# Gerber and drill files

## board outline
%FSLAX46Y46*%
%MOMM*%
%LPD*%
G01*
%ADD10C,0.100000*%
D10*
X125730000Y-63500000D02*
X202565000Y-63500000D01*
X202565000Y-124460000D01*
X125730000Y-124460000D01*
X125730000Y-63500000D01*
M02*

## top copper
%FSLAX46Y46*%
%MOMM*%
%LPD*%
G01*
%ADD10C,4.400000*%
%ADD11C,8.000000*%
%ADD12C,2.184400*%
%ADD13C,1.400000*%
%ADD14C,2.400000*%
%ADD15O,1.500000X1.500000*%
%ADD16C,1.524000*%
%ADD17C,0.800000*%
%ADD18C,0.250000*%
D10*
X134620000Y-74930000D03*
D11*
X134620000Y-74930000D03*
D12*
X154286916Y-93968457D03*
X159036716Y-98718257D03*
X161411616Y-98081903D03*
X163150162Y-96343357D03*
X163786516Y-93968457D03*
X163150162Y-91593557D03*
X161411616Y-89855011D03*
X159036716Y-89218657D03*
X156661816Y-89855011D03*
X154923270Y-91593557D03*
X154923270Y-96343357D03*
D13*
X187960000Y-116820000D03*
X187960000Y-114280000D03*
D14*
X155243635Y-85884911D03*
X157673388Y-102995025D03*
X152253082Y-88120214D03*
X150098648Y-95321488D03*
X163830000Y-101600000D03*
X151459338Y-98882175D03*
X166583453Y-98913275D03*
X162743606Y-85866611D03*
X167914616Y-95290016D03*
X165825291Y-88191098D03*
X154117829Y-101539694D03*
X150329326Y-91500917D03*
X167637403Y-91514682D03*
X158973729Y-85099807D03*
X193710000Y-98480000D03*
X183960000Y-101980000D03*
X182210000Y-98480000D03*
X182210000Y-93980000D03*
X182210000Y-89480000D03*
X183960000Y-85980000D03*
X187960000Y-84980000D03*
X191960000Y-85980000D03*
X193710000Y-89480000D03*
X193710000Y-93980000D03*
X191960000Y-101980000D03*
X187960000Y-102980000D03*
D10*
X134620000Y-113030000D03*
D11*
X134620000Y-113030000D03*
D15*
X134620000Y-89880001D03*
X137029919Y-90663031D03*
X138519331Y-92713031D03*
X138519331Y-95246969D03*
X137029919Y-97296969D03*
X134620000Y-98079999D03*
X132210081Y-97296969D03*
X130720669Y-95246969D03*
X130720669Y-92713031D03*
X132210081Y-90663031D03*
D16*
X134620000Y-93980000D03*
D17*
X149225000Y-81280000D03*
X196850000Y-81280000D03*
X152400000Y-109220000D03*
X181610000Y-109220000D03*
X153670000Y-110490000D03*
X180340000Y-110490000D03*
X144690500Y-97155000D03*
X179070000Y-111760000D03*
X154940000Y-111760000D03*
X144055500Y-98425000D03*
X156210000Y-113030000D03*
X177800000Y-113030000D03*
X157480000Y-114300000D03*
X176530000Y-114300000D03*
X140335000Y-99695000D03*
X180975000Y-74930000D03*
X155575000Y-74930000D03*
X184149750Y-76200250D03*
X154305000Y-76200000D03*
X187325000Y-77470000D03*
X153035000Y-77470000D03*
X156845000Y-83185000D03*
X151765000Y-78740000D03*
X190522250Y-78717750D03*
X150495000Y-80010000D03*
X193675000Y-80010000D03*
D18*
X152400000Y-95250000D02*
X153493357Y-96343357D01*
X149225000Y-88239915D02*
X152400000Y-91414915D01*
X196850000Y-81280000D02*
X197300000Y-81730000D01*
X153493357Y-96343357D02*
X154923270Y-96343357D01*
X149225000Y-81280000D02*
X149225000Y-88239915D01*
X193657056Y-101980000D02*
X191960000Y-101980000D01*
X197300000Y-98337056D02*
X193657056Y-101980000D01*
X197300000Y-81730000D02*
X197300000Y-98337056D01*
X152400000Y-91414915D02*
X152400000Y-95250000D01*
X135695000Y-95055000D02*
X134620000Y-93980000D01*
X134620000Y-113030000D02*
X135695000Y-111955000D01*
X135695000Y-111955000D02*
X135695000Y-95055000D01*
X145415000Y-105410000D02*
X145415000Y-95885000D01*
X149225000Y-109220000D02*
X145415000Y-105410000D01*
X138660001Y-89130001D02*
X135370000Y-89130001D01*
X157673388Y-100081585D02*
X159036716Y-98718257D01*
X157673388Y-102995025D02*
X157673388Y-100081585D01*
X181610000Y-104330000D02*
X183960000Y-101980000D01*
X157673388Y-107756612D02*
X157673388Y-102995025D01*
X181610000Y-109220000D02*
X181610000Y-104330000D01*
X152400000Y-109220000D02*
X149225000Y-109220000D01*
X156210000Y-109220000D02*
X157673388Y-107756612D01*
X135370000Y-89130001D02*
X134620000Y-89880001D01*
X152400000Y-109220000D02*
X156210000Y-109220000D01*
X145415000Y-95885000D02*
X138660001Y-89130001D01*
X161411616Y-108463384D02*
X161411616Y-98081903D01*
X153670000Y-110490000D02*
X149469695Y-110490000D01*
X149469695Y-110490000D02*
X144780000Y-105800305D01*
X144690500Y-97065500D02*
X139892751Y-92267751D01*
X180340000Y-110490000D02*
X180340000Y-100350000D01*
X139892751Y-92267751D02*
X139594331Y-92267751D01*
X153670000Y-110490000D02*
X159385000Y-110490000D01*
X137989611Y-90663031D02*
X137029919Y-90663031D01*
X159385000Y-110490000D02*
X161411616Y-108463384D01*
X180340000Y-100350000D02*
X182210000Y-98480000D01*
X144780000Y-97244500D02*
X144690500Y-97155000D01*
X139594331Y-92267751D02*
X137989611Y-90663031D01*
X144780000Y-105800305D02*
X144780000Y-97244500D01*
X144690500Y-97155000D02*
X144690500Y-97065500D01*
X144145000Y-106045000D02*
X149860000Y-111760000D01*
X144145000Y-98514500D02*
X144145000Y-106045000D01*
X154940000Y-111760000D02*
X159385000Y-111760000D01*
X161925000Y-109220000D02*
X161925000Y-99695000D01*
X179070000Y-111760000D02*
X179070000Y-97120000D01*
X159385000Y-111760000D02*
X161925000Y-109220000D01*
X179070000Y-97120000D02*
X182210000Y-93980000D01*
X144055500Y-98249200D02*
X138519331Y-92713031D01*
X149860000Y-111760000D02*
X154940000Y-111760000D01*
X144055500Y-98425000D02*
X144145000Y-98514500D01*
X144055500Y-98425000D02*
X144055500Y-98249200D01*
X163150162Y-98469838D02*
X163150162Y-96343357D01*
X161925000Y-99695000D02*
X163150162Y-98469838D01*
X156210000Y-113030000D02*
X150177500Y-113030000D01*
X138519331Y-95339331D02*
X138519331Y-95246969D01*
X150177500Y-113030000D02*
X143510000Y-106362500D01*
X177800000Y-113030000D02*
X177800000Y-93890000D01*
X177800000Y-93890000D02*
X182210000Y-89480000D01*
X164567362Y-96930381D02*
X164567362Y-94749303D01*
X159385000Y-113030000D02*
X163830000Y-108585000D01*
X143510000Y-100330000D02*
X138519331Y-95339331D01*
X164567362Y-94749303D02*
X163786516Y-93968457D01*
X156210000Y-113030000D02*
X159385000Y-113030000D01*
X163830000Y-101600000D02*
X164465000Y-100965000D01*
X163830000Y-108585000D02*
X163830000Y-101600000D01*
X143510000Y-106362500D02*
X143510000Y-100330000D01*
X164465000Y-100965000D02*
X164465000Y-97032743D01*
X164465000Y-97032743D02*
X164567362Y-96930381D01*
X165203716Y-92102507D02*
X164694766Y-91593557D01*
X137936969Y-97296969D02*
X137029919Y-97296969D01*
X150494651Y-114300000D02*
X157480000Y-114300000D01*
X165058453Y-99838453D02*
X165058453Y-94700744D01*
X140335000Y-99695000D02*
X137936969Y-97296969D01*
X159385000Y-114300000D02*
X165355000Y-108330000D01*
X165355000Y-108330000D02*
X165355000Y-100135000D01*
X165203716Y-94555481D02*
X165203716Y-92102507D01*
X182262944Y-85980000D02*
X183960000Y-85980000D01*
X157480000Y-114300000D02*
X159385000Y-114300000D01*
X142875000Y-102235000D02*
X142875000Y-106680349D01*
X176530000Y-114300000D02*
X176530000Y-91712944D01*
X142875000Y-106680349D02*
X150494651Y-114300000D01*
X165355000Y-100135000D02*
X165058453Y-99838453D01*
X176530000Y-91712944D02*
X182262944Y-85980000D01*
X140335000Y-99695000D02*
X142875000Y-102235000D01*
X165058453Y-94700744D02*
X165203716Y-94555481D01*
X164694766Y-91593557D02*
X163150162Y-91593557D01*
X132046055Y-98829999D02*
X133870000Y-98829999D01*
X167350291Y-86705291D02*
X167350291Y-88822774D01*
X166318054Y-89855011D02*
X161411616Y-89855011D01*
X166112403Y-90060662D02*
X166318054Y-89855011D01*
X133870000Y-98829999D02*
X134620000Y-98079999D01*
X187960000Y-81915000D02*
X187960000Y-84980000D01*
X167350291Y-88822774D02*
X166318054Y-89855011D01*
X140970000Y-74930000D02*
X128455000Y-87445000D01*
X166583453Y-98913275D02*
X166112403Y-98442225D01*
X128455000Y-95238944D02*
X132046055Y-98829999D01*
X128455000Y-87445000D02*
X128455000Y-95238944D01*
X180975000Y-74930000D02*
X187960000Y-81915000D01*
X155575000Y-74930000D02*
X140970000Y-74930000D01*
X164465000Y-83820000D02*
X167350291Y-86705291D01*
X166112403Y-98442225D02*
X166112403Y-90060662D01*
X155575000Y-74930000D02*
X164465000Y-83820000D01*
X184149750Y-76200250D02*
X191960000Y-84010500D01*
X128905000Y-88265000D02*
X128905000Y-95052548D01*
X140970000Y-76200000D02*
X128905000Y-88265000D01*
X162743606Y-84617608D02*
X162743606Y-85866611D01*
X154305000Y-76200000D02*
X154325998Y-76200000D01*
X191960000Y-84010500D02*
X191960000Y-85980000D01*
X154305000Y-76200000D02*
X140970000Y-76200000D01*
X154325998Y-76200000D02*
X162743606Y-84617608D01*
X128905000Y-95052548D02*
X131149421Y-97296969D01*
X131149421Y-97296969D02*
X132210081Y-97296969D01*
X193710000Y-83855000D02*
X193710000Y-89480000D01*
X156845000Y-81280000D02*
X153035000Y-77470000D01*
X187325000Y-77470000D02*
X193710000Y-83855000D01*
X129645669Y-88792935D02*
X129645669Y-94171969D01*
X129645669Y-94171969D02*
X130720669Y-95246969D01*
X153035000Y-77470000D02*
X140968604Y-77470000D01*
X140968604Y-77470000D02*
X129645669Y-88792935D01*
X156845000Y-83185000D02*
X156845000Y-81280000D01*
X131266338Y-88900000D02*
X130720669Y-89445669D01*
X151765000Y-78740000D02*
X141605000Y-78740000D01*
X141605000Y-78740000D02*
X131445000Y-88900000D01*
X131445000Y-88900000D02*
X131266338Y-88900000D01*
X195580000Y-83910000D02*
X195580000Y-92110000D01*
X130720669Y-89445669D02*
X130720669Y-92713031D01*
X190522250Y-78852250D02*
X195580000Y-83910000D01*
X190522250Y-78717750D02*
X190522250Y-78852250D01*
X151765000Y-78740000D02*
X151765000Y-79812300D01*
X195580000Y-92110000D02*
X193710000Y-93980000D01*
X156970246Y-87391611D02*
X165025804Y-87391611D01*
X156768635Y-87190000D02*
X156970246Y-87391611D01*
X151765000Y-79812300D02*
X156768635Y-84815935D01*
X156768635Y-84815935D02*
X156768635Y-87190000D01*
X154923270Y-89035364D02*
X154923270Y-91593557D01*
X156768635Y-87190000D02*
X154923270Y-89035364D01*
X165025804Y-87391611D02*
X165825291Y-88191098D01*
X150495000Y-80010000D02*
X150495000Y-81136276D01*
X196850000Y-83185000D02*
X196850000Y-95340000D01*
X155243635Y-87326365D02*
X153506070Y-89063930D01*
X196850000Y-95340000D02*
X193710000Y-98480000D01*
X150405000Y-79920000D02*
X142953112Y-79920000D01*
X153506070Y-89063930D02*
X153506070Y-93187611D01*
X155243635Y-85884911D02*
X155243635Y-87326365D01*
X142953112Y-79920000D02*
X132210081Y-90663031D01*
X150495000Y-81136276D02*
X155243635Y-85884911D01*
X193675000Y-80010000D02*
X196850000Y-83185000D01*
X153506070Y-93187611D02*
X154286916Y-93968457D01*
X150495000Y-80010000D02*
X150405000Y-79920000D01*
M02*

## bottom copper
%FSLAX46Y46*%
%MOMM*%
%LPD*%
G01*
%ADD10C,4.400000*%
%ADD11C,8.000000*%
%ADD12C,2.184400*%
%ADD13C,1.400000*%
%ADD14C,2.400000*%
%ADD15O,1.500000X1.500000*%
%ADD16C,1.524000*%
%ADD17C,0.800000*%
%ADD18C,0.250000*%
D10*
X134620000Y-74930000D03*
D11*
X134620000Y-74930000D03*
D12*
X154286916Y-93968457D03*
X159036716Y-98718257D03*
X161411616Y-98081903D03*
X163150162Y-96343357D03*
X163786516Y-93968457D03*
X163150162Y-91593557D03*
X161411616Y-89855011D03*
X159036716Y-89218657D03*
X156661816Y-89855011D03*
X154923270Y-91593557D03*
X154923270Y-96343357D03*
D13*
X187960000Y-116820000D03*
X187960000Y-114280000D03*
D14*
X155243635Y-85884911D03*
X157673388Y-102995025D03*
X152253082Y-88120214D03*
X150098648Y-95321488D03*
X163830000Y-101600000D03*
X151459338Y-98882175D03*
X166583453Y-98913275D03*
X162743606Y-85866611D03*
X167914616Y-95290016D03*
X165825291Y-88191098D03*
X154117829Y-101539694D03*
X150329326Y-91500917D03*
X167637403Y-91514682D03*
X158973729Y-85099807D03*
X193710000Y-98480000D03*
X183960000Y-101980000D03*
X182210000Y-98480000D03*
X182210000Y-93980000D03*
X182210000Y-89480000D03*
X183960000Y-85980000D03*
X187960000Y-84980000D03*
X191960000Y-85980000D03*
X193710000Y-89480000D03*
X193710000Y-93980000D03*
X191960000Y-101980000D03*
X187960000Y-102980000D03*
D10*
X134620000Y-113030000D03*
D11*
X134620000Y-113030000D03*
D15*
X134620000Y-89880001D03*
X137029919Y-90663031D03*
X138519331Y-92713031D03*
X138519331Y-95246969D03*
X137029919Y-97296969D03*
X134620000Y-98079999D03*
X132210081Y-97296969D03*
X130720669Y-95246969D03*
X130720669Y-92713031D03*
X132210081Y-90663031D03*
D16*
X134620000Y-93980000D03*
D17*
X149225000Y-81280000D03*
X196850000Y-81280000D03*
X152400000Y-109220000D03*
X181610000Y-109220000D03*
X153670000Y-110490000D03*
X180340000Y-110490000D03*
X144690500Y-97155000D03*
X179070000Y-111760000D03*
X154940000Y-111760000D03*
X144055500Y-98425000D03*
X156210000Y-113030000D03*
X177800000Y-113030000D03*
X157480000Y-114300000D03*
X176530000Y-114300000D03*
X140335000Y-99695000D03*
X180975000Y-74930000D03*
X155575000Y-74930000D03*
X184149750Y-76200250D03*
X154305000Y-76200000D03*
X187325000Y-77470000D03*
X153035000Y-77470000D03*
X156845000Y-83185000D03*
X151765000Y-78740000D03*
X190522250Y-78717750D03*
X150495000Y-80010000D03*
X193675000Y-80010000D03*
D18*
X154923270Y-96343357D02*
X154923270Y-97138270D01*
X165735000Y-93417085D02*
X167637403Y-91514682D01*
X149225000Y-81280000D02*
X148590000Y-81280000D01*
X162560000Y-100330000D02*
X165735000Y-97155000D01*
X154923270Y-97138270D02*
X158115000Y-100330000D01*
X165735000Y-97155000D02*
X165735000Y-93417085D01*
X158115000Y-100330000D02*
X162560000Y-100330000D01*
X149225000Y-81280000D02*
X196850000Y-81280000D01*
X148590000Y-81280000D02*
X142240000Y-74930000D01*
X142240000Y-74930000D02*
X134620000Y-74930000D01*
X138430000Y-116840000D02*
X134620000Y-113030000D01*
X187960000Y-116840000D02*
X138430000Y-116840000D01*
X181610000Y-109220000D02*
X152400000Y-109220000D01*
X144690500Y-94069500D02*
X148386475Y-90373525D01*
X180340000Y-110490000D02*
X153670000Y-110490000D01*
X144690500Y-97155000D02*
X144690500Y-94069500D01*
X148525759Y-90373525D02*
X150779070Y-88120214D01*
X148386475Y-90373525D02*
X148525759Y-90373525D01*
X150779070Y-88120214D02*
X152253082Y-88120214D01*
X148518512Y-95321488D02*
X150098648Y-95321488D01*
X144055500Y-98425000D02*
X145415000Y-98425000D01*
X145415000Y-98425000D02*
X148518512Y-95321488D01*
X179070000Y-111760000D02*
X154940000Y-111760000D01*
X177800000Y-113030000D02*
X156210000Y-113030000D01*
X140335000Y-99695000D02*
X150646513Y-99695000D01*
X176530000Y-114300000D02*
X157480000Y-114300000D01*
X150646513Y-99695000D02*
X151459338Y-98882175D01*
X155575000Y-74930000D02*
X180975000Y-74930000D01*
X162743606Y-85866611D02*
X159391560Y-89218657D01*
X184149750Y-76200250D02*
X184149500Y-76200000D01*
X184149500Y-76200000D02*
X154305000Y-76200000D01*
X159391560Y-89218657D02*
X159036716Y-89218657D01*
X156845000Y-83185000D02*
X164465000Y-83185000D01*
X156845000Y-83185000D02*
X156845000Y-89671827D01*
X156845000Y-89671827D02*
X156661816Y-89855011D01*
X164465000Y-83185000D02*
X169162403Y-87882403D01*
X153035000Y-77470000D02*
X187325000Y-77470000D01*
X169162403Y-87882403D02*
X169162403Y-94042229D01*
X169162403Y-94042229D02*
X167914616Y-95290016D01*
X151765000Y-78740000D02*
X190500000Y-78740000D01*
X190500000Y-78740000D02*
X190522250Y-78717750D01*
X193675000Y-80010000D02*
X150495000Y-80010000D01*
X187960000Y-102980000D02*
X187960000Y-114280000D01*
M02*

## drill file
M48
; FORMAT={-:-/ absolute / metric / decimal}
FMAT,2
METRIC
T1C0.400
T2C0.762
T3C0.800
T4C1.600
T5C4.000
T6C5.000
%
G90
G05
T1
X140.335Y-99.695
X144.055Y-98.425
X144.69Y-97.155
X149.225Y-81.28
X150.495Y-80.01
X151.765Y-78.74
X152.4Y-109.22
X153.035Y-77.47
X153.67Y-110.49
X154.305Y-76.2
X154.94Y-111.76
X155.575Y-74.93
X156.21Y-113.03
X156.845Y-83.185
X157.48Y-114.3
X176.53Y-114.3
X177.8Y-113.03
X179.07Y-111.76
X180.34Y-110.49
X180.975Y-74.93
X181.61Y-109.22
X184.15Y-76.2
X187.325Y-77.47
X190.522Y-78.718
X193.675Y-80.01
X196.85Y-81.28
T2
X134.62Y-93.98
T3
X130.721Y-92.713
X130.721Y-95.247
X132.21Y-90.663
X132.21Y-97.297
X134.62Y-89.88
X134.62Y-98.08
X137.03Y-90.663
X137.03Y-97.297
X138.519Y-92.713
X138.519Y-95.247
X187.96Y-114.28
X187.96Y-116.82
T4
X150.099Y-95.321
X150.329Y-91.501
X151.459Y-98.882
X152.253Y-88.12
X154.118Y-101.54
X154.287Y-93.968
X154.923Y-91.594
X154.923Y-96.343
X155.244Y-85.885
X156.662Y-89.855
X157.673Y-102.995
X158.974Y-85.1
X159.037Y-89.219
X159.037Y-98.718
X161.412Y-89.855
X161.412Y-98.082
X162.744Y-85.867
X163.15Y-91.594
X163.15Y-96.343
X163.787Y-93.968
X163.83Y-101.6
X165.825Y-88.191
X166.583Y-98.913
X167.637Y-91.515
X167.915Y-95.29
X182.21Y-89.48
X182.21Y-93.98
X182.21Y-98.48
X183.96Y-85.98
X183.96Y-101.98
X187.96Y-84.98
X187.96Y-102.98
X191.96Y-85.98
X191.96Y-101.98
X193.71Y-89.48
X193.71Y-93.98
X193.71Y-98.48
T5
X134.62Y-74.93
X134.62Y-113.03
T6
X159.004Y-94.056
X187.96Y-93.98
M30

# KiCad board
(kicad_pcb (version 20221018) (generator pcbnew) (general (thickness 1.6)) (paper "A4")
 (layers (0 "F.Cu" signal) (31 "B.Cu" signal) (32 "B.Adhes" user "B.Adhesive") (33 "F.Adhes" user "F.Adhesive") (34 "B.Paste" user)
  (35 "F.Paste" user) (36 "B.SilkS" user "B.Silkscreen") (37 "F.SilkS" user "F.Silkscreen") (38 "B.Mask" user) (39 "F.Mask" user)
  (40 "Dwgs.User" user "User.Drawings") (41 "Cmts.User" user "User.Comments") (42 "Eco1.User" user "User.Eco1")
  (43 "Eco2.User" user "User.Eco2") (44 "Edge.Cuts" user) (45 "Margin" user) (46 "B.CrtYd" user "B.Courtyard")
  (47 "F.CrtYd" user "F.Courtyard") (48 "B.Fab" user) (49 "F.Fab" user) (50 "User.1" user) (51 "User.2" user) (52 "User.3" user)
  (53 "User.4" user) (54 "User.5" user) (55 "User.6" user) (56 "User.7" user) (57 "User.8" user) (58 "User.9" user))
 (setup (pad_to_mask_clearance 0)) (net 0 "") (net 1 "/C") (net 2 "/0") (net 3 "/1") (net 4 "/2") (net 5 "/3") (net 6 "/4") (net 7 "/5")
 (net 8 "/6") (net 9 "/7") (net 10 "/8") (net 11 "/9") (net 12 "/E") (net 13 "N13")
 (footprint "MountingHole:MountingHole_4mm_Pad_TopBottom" (layer "F.Cu") (at 134.62 74.93)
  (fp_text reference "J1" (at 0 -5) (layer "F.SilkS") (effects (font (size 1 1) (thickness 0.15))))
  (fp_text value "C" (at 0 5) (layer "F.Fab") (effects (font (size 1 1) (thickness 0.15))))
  (pad "1" thru_hole circle (at 0 0) (size 4.4 4.4) (drill 4) (layers "*.Cu" "*.Mask") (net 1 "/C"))
  (pad "1" connect circle (at 0 0) (size 8 8) (layers "F.Cu" "F.Mask") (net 1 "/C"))
  (pad "1" connect circle (at 0 0) (size 8 8) (layers "B.Cu" "B.Mask") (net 1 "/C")))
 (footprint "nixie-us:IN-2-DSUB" (layer "F.Cu") (at 159.036716 93.968457)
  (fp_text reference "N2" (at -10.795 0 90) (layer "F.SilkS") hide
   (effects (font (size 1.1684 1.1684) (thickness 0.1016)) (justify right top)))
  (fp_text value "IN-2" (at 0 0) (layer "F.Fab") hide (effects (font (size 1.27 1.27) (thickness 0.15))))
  (pad "0" thru_hole circle (at -4.7498 0 180) (size 2.1844 2.1844) (drill 1.6) (layers "*.Cu" "*.Mask") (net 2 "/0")
   (solder_mask_margin 0.1016))
  (pad "1" thru_hole circle (at 0 4.7498 270) (size 2.1844 2.1844) (drill 1.6) (layers "*.Cu" "*.Mask") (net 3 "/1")
   (solder_mask_margin 0.1016))
  (pad "2" thru_hole circle (at 2.3749 4.113446 300) (size 2.1844 2.1844) (drill 1.6) (layers "*.Cu" "*.Mask") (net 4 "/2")
   (solder_mask_margin 0.1016))
  (pad "3" thru_hole circle (at 4.113446 2.3749 330) (size 2.1844 2.1844) (drill 1.6) (layers "*.Cu" "*.Mask") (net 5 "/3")
   (solder_mask_margin 0.1016))
  (pad "4" thru_hole circle (at 4.7498 0) (size 2.1844 2.1844) (drill 1.6) (layers "*.Cu" "*.Mask") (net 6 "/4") (solder_mask_margin 0.1016))
  (pad "5" thru_hole circle (at 4.113446 -2.3749 30) (size 2.1844 2.1844) (drill 1.6) (layers "*.Cu" "*.Mask") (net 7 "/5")
   (solder_mask_margin 0.1016))
  (pad "6" thru_hole circle (at 2.3749 -4.113446 60) (size 2.1844 2.1844) (drill 1.6) (layers "*.Cu" "*.Mask") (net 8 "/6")
   (solder_mask_margin 0.1016))
  (pad "7" thru_hole circle (at 0 -4.7498 90) (size 2.1844 2.1844) (drill 1.6) (layers "*.Cu" "*.Mask") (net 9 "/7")
   (solder_mask_margin 0.1016))
  (pad "8" thru_hole circle (at -2.3749 -4.113446 120) (size 2.1844 2.1844) (drill 1.6) (layers "*.Cu" "*.Mask") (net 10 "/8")
   (solder_mask_margin 0.1016))
  (pad "9" thru_hole circle (at -4.113446 -2.3749 150) (size 2.1844 2.1844) (drill 1.6) (layers "*.Cu" "*.Mask") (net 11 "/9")
   (solder_mask_margin 0.1016))
  (pad "A" thru_hole circle (at -4.113446 2.3749 210) (size 2.1844 2.1844) (drill 1.6) (layers "*.Cu" "*.Mask") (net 1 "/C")
   (solder_mask_margin 0.1016)))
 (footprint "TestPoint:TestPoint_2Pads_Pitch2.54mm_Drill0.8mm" (layer "F.Cu") (at 187.96 116.82 90)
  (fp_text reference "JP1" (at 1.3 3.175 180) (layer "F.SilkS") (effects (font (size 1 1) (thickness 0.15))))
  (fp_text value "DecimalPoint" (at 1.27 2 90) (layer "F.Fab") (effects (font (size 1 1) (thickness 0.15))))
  (pad "1" thru_hole circle (at 0 0 90) (size 1.4 1.4) (drill 0.8) (layers "*.Cu" "*.Mask") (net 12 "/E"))
  (pad "2" thru_hole circle (at 2.54 0 90) (size 1.4 1.4) (drill 0.8) (layers "*.Cu" "*.Mask") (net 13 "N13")))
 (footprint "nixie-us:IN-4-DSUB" (layer "F.Cu") (at 159.036716 93.968457)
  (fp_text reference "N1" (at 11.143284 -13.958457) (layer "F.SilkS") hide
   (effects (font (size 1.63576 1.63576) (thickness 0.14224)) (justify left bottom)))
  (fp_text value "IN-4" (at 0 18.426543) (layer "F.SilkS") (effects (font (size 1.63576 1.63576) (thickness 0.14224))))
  (pad "" np_thru_hole circle (at -0.033137 0.0873) (size 5 5) (drill 5) (layers "*.Cu" "*.Mask"))
  (pad "0" thru_hole circle (at -3.793081 -8.083546) (size 2.4 2.4) (drill 1.6) (layers "*.Cu" "*.Mask") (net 2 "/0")
   (solder_mask_margin 0.1016))
  (pad "1" thru_hole circle (at -1.363328 9.026568) (size 2.4 2.4) (drill 1.6) (layers "*.Cu" "*.Mask") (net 3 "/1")
   (solder_mask_margin 0.1016))
  (pad "2" thru_hole circle (at -6.783634 -5.848243) (size 2.4 2.4) (drill 1.6) (layers "*.Cu" "*.Mask") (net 4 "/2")
   (solder_mask_margin 0.1016))
  (pad "3" thru_hole circle (at -8.938068 1.353031) (size 2.4 2.4) (drill 1.6) (layers "*.Cu" "*.Mask") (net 5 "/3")
   (solder_mask_margin 0.1016))
  (pad "4" thru_hole circle (at 4.793284 7.631543) (size 2.4 2.4) (drill 1.6) (layers "*.Cu" "*.Mask") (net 6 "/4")
   (solder_mask_margin 0.1016))
  (pad "5" thru_hole circle (at -7.577378 4.913718) (size 2.4 2.4) (drill 1.6) (layers "*.Cu" "*.Mask") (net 7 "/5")
   (solder_mask_margin 0.1016))
  (pad "6" thru_hole circle (at 7.546737 4.944818) (size 2.4 2.4) (drill 1.6) (layers "*.Cu" "*.Mask") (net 8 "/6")
   (solder_mask_margin 0.1016))
  (pad "7" thru_hole circle (at 3.70689 -8.101846) (size 2.4 2.4) (drill 1.6) (layers "*.Cu" "*.Mask") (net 9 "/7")
   (solder_mask_margin 0.1016))
  (pad "8" thru_hole circle (at 8.8779 1.321559) (size 2.4 2.4) (drill 1.6) (layers "*.Cu" "*.Mask") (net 10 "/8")
   (solder_mask_margin 0.1016))
  (pad "9" thru_hole circle (at 6.788575 -5.777359) (size 2.4 2.4) (drill 1.6) (layers "*.Cu" "*.Mask") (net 11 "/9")
   (solder_mask_margin 0.1016))
  (pad "A1" thru_hole circle (at -4.918887 7.571237) (size 2.4 2.4) (drill 1.6) (layers "*.Cu" "*.Mask") (solder_mask_margin 0.1016))
  (pad "A2" thru_hole circle (at -8.70739 -2.46754) (size 2.4 2.4) (drill 1.6) (layers "*.Cu" "*.Mask") (solder_mask_margin 0.1016))
  (pad "A3" thru_hole circle (at 8.600687 -2.453775) (size 2.4 2.4) (drill 1.6) (layers "*.Cu" "*.Mask") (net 1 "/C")
   (solder_mask_margin 0.1016))
  (pad "N/C" thru_hole circle (at -0.062987 -8.86865) (size 2.4 2.4) (drill 1.6) (layers "*.Cu" "*.Mask") (solder_mask_margin 0.1016)))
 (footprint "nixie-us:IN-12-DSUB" (layer "F.Cu") (at 187.96 93.98)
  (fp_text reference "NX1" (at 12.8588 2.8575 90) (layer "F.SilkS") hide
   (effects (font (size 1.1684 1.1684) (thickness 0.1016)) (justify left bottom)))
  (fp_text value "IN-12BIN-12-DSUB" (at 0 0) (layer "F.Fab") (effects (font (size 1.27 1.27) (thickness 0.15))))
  (pad "" np_thru_hole circle (at 0 0) (size 5 5) (drill 5) (layers "*.Cu" "*.Mask"))
  (pad "0" thru_hole circle (at 5.75 4.5) (size 2.4 2.4) (drill 1.6) (layers "*.Cu" "*.Mask") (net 2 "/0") (solder_mask_margin 0.1016))
  (pad "1" thru_hole circle (at -4 8) (size 2.4 2.4) (drill 1.6) (layers "*.Cu" "*.Mask") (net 3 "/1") (solder_mask_margin 0.1016))
  (pad "2" thru_hole circle (at -5.75 4.5) (size 2.4 2.4) (drill 1.6) (layers "*.Cu" "*.Mask") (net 4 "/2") (solder_mask_margin 0.1016))
  (pad "3" thru_hole circle (at -5.75 0) (size 2.4 2.4) (drill 1.6) (layers "*.Cu" "*.Mask") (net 5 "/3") (solder_mask_margin 0.1016))
  (pad "4" thru_hole circle (at -5.75 -4.5) (size 2.4 2.4) (drill 1.6) (layers "*.Cu" "*.Mask") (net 6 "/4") (solder_mask_margin 0.1016))
  (pad "5" thru_hole circle (at -4 -8) (size 2.4 2.4) (drill 1.6) (layers "*.Cu" "*.Mask") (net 7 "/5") (solder_mask_margin 0.1016))
  (pad "6" thru_hole circle (at 0 -9) (size 2.4 2.4) (drill 1.6) (layers "*.Cu" "*.Mask") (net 8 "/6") (solder_mask_margin 0.1016))
  (pad "7" thru_hole circle (at 4 -8) (size 2.4 2.4) (drill 1.6) (layers "*.Cu" "*.Mask") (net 9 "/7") (solder_mask_margin 0.1016))
  (pad "8" thru_hole circle (at 5.75 -4.5) (size 2.4 2.4) (drill 1.6) (layers "*.Cu" "*.Mask") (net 10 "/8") (solder_mask_margin 0.1016))
  (pad "9" thru_hole circle (at 5.75 0) (size 2.4 2.4) (drill 1.6) (layers "*.Cu" "*.Mask") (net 11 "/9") (solder_mask_margin 0.1016))
  (pad "A" thru_hole circle (at 4 8) (size 2.4 2.4) (drill 1.6) (layers "*.Cu" "*.Mask") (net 1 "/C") (solder_mask_margin 0.1016))
  (pad "LHDP" thru_hole circle (at 0 9) (size 2.4 2.4) (drill 1.6) (layers "*.Cu" "*.Mask") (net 13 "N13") (solder_mask_margin 0.1016)))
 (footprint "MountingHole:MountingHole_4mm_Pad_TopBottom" (layer "F.Cu") (at 134.62 113.03)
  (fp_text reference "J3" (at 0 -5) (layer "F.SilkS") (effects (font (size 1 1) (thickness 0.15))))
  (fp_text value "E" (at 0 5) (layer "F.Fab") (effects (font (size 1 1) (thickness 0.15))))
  (pad "1" thru_hole circle (at 0 0) (size 4.4 4.4) (drill 4) (layers "*.Cu" "*.Mask") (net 12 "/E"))
  (pad "1" connect circle (at 0 0) (size 8 8) (layers "F.Cu" "F.Mask") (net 12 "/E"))
  (pad "1" connect circle (at 0 0) (size 8 8) (layers "B.Cu" "B.Mask") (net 12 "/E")))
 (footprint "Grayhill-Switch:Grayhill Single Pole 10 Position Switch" (layer "F.Cu") (at 134.62 93.98)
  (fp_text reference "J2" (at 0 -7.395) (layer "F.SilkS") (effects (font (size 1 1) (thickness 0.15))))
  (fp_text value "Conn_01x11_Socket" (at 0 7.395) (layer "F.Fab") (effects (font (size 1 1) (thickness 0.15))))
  (pad "1" thru_hole oval (at 0 -4.099999) (size 1.5 1.5) (drill 0.8) (layers "*.Cu" "*.Mask") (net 3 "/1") (thermal_bridge_angle 45))
  (pad "2" thru_hole oval (at 2.409919 -3.316969) (size 1.5 1.5) (drill 0.8) (layers "*.Cu" "*.Mask") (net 4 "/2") (thermal_bridge_angle 45))
  (pad "3" thru_hole oval (at 3.899331 -1.266969) (size 1.5 1.5) (drill 0.8) (layers "*.Cu" "*.Mask") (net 5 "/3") (thermal_bridge_angle 45))
  (pad "4" thru_hole oval (at 3.899331 1.266969) (size 1.5 1.5) (drill 0.8) (layers "*.Cu" "*.Mask") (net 6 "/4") (thermal_bridge_angle 45))
  (pad "5" thru_hole oval (at 2.409919 3.316969) (size 1.5 1.5) (drill 0.8) (layers "*.Cu" "*.Mask") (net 7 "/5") (thermal_bridge_angle 45))
  (pad "6" thru_hole oval (at 0 4.099999) (size 1.5 1.5) (drill 0.8) (layers "*.Cu" "*.Mask") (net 8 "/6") (thermal_bridge_angle 45))
  (pad "7" thru_hole oval (at -2.409919 3.316969) (size 1.5 1.5) (drill 0.8) (layers "*.Cu" "*.Mask") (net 9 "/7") (thermal_bridge_angle 45))
  (pad "8" thru_hole oval (at -3.899331 1.266969) (size 1.5 1.5) (drill 0.8) (layers "*.Cu" "*.Mask") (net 10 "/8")
   (thermal_bridge_angle 45))
  (pad "9" thru_hole oval (at -3.899331 -1.266969) (size 1.5 1.5) (drill 0.8) (layers "*.Cu" "*.Mask") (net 11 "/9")
   (thermal_bridge_angle 45))
  (pad "10" thru_hole oval (at -2.409919 -3.316969) (size 1.5 1.5) (drill 0.8) (layers "*.Cu" "*.Mask") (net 2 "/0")
   (thermal_bridge_angle 45))
  (pad "11" thru_hole circle (at 0 0) (size 1.524 1.524) (drill 0.762) (layers "*.Cu" "*.Mask") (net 12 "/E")))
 (gr_rect (start 125.73 63.5) (end 202.565 124.46) (stroke (width 0.1) (type default)) (fill none) (layer "Edge.Cuts"))
 (segment (start 152.4 95.25) (end 153.493357 96.343357) (width 0.25) (layer "F.Cu") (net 1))
 (segment (start 149.225 88.239915) (end 152.4 91.414915) (width 0.25) (layer "F.Cu") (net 1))
 (segment (start 196.85 81.28) (end 197.3 81.73) (width 0.25) (layer "F.Cu") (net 1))
 (segment (start 153.493357 96.343357) (end 154.92327 96.343357) (width 0.25) (layer "F.Cu") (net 1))
 (segment (start 149.225 81.28) (end 149.225 88.239915) (width 0.25) (layer "F.Cu") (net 1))
 (segment (start 193.657056 101.98) (end 191.96 101.98) (width 0.25) (layer "F.Cu") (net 1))
 (segment (start 197.3 98.337056) (end 193.657056 101.98) (width 0.25) (layer "F.Cu") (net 1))
 (segment (start 197.3 81.73) (end 197.3 98.337056) (width 0.25) (layer "F.Cu") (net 1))
 (segment (start 152.4 91.414915) (end 152.4 95.25) (width 0.25) (layer "F.Cu") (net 1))
 (via (at 149.225 81.28) (size 0.8) (drill 0.4) (layers "F.Cu" "B.Cu") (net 1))
 (via (at 196.85 81.28) (size 0.8) (drill 0.4) (layers "F.Cu" "B.Cu") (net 1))
 (segment (start 154.92327 96.343357) (end 154.92327 97.13827) (width 0.25) (layer "B.Cu") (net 1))
 (segment (start 165.735 93.417085) (end 167.637403 91.514682) (width 0.25) (layer "B.Cu") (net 1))
 (segment (start 149.225 81.28) (end 148.59 81.28) (width 0.25) (layer "B.Cu") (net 1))
 (segment (start 162.56 100.33) (end 165.735 97.155) (width 0.25) (layer "B.Cu") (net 1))
 (segment (start 154.92327 97.13827) (end 158.115 100.33) (width 0.25) (layer "B.Cu") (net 1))
 (segment (start 165.735 97.155) (end 165.735 93.417085) (width 0.25) (layer "B.Cu") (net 1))
 (segment (start 158.115 100.33) (end 162.56 100.33) (width 0.25) (layer "B.Cu") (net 1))
 (segment (start 149.225 81.28) (end 196.85 81.28) (width 0.25) (layer "B.Cu") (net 1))
 (segment (start 148.59 81.28) (end 142.24 74.93) (width 0.25) (layer "B.Cu") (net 1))
 (segment (start 142.24 74.93) (end 134.62 74.93) (width 0.25) (layer "B.Cu") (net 1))
 (segment (start 135.695 95.055) (end 134.62 93.98) (width 0.25) (layer "F.Cu") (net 12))
 (segment (start 134.62 113.03) (end 135.695 111.955) (width 0.25) (layer "F.Cu") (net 12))
 (segment (start 135.695 111.955) (end 135.695 95.055) (width 0.25) (layer "F.Cu") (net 12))
 (segment (start 138.43 116.84) (end 134.62 113.03) (width 0.25) (layer "B.Cu") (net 12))
 (segment (start 187.96 116.84) (end 138.43 116.84) (width 0.25) (layer "B.Cu") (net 12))
 (segment (start 145.415 105.41) (end 145.415 95.885) (width 0.25) (layer "F.Cu") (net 3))
 (segment (start 149.225 109.22) (end 145.415 105.41) (width 0.25) (layer "F.Cu") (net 3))
 (segment (start 138.660001 89.130001) (end 135.37 89.130001) (width 0.25) (layer "F.Cu") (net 3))
 (segment (start 157.673388 100.081585) (end 159.036716 98.718257) (width 0.25) (layer "F.Cu") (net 3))
 (segment (start 157.673388 102.995025) (end 157.673388 100.081585) (width 0.25) (layer "F.Cu") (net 3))
 (segment (start 181.61 104.33) (end 183.96 101.98) (width 0.25) (layer "F.Cu") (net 3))
 (segment (start 157.673388 107.756612) (end 157.673388 102.995025) (width 0.25) (layer "F.Cu") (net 3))
 (segment (start 181.61 109.22) (end 181.61 104.33) (width 0.25) (layer "F.Cu") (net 3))
 (segment (start 152.4 109.22) (end 149.225 109.22) (width 0.25) (layer "F.Cu") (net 3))
 (segment (start 156.21 109.22) (end 157.673388 107.756612) (width 0.25) (layer "F.Cu") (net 3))
 (segment (start 135.37 89.130001) (end 134.62 89.880001) (width 0.25) (layer "F.Cu") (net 3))
 (segment (start 152.4 109.22) (end 156.21 109.22) (width 0.25) (layer "F.Cu") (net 3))
 (segment (start 145.415 95.885) (end 138.660001 89.130001) (width 0.25) (layer "F.Cu") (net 3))
 (via (at 152.4 109.22) (size 0.8) (drill 0.4) (layers "F.Cu" "B.Cu") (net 3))
 (via (at 181.61 109.22) (size 0.8) (drill 0.4) (layers "F.Cu" "B.Cu") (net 3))
 (segment (start 181.61 109.22) (end 152.4 109.22) (width 0.25) (layer "B.Cu") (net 3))
 (segment (start 161.411616 108.463384) (end 161.411616 98.081903) (width 0.25) (layer "F.Cu") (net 4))
 (segment (start 153.67 110.49) (end 149.469695 110.49) (width 0.25) (layer "F.Cu") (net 4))
 (segment (start 149.469695 110.49) (end 144.78 105.800305) (width 0.25) (layer "F.Cu") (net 4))
 (segment (start 144.6905 97.0655) (end 139.892751 92.267751) (width 0.25) (layer "F.Cu") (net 4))
 (segment (start 180.34 110.49) (end 180.34 100.35) (width 0.25) (layer "F.Cu") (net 4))
 (segment (start 139.892751 92.267751) (end 139.594331 92.267751) (width 0.25) (layer "F.Cu") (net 4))
 (segment (start 153.67 110.49) (end 159.385 110.49) (width 0.25) (layer "F.Cu") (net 4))
 (segment (start 137.989611 90.663031) (end 137.029919 90.663031) (width 0.25) (layer "F.Cu") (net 4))
 (segment (start 159.385 110.49) (end 161.411616 108.463384) (width 0.25) (layer "F.Cu") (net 4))
 (segment (start 180.34 100.35) (end 182.21 98.48) (width 0.25) (layer "F.Cu") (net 4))
 (segment (start 144.78 97.2445) (end 144.6905 97.155) (width 0.25) (layer "F.Cu") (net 4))
 (segment (start 139.594331 92.267751) (end 137.989611 90.663031) (width 0.25) (layer "F.Cu") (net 4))
 (segment (start 144.78 105.800305) (end 144.78 97.2445) (width 0.25) (layer "F.Cu") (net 4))
 (segment (start 144.6905 97.155) (end 144.6905 97.0655) (width 0.25) (layer "F.Cu") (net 4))
 (via (at 153.67 110.49) (size 0.8) (drill 0.4) (layers "F.Cu" "B.Cu") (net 4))
 (via (at 180.34 110.49) (size 0.8) (drill 0.4) (layers "F.Cu" "B.Cu") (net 4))
 (via (at 144.6905 97.155) (size 0.8) (drill 0.4) (layers "F.Cu" "B.Cu") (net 4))
 (segment (start 144.6905 94.0695) (end 148.386475 90.373525) (width 0.25) (layer "B.Cu") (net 4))
 (segment (start 180.34 110.49) (end 153.67 110.49) (width 0.25) (layer "B.Cu") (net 4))
 (segment (start 144.6905 97.155) (end 144.6905 94.0695) (width 0.25) (layer "B.Cu") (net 4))
 (segment (start 148.525759 90.373525) (end 150.77907 88.120214) (width 0.25) (layer "B.Cu") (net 4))
 (segment (start 148.386475 90.373525) (end 148.525759 90.373525) (width 0.25) (layer "B.Cu") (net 4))
 (segment (start 150.77907 88.120214) (end 152.253082 88.120214) (width 0.25) (layer "B.Cu") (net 4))
 (segment (start 144.145 106.045) (end 149.86 111.76) (width 0.25) (layer "F.Cu") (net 5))
 (segment (start 144.145 98.5145) (end 144.145 106.045) (width 0.25) (layer "F.Cu") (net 5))
 (segment (start 154.94 111.76) (end 159.385 111.76) (width 0.25) (layer "F.Cu") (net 5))
 (segment (start 161.925 109.22) (end 161.925 99.695) (width 0.25) (layer "F.Cu") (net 5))
 (segment (start 179.07 111.76) (end 179.07 97.12) (width 0.25) (layer "F.Cu") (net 5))
 (segment (start 159.385 111.76) (end 161.925 109.22) (width 0.25) (layer "F.Cu") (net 5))
 (segment (start 179.07 97.12) (end 182.21 93.98) (width 0.25) (layer "F.Cu") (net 5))
 (segment (start 144.0555 98.2492) (end 138.519331 92.713031) (width 0.25) (layer "F.Cu") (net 5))
 (segment (start 149.86 111.76) (end 154.94 111.76) (width 0.25) (layer "F.Cu") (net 5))
 (segment (start 144.0555 98.425) (end 144.145 98.5145) (width 0.25) (layer "F.Cu") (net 5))
 (segment (start 144.0555 98.425) (end 144.0555 98.2492) (width 0.25) (layer "F.Cu") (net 5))
 (segment (start 163.150162 98.469838) (end 163.150162 96.343357) (width 0.25) (layer "F.Cu") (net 5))
 (segment (start 161.925 99.695) (end 163.150162 98.469838) (width 0.25) (layer "F.Cu") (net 5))
 (via (at 179.07 111.76) (size 0.8) (drill 0.4) (layers "F.Cu" "B.Cu") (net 5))
 (via (at 154.94 111.76) (size 0.8) (drill 0.4) (layers "F.Cu" "B.Cu") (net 5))
 (via (at 144.0555 98.425) (size 0.8) (drill 0.4) (layers "F.Cu" "B.Cu") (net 5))
 (segment (start 148.518512 95.321488) (end 150.098648 95.321488) (width 0.25) (layer "B.Cu") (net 5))
 (segment (start 144.0555 98.425) (end 145.415 98.425) (width 0.25) (layer "B.Cu") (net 5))
 (segment (start 145.415 98.425) (end 148.518512 95.321488) (width 0.25) (layer "B.Cu") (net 5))
 (segment (start 179.07 111.76) (end 154.94 111.76) (width 0.25) (layer "B.Cu") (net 5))
 (segment (start 156.21 113.03) (end 150.1775 113.03) (width 0.25) (layer "F.Cu") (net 6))
 (segment (start 138.519331 95.339331) (end 138.519331 95.246969) (width 0.25) (layer "F.Cu") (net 6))
 (segment (start 150.1775 113.03) (end 143.51 106.3625) (width 0.25) (layer "F.Cu") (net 6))
 (segment (start 177.8 113.03) (end 177.8 93.89) (width 0.25) (layer "F.Cu") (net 6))
 (segment (start 177.8 93.89) (end 182.21 89.48) (width 0.25) (layer "F.Cu") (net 6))
 (segment (start 164.567362 96.930381) (end 164.567362 94.749303) (width 0.25) (layer "F.Cu") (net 6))
 (segment (start 159.385 113.03) (end 163.83 108.585) (width 0.25) (layer "F.Cu") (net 6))
 (segment (start 143.51 100.33) (end 138.519331 95.339331) (width 0.25) (layer "F.Cu") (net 6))
 (segment (start 164.567362 94.749303) (end 163.786516 93.968457) (width 0.25) (layer "F.Cu") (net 6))
 (segment (start 156.21 113.03) (end 159.385 113.03) (width 0.25) (layer "F.Cu") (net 6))
 (segment (start 163.83 101.6) (end 164.465 100.965) (width 0.25) (layer "F.Cu") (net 6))
 (segment (start 163.83 108.585) (end 163.83 101.6) (width 0.25) (layer "F.Cu") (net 6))
 (segment (start 143.51 106.3625) (end 143.51 100.33) (width 0.25) (layer "F.Cu") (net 6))
 (segment (start 164.465 100.965) (end 164.465 97.032743) (width 0.25) (layer "F.Cu") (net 6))
 (segment (start 164.465 97.032743) (end 164.567362 96.930381) (width 0.25) (layer "F.Cu") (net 6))
 (via (at 156.21 113.03) (size 0.8) (drill 0.4) (layers "F.Cu" "B.Cu") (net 6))
 (via (at 177.8 113.03) (size 0.8) (drill 0.4) (layers "F.Cu" "B.Cu") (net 6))
 (segment (start 177.8 113.03) (end 156.21 113.03) (width 0.25) (layer "B.Cu") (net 6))
 (segment (start 165.203716 92.102507) (end 164.694766 91.593557) (width 0.25) (layer "F.Cu") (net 7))
 (segment (start 137.936969 97.296969) (end 137.029919 97.296969) (width 0.25) (layer "F.Cu") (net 7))
 (segment (start 150.494651 114.3) (end 157.48 114.3) (width 0.25) (layer "F.Cu") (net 7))
 (segment (start 165.058453 99.838453) (end 165.058453 94.700744) (width 0.25) (layer "F.Cu") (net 7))
 (segment (start 140.335 99.695) (end 137.936969 97.296969) (width 0.25) (layer "F.Cu") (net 7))
 (segment (start 159.385 114.3) (end 165.355 108.33) (width 0.25) (layer "F.Cu") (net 7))
 (segment (start 165.355 108.33) (end 165.355 100.135) (width 0.25) (layer "F.Cu") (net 7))
 (segment (start 165.203716 94.555481) (end 165.203716 92.102507) (width 0.25) (layer "F.Cu") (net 7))
 (segment (start 182.262944 85.98) (end 183.96 85.98) (width 0.25) (layer "F.Cu") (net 7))
 (segment (start 157.48 114.3) (end 159.385 114.3) (width 0.25) (layer "F.Cu") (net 7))
 (segment (start 142.875 102.235) (end 142.875 106.680349) (width 0.25) (layer "F.Cu") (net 7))
 (segment (start 176.53 114.3) (end 176.53 91.712944) (width 0.25) (layer "F.Cu") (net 7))
 (segment (start 142.875 106.680349) (end 150.494651 114.3) (width 0.25) (layer "F.Cu") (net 7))
 (segment (start 165.355 100.135) (end 165.058453 99.838453) (width 0.25) (layer "F.Cu") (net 7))
 (segment (start 176.53 91.712944) (end 182.262944 85.98) (width 0.25) (layer "F.Cu") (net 7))
 (segment (start 140.335 99.695) (end 142.875 102.235) (width 0.25) (layer "F.Cu") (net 7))
 (segment (start 165.058453 94.700744) (end 165.203716 94.555481) (width 0.25) (layer "F.Cu") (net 7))
 (segment (start 164.694766 91.593557) (end 163.150162 91.593557) (width 0.25) (layer "F.Cu") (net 7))
 (via (at 157.48 114.3) (size 0.8) (drill 0.4) (layers "F.Cu" "B.Cu") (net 7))
 (via (at 176.53 114.3) (size 0.8) (drill 0.4) (layers "F.Cu" "B.Cu") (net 7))
 (via (at 140.335 99.695) (size 0.8) (drill 0.4) (layers "F.Cu" "B.Cu") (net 7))
 (segment (start 140.335 99.695) (end 150.646513 99.695) (width 0.25) (layer "B.Cu") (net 7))
 (segment (start 176.53 114.3) (end 157.48 114.3) (width 0.25) (layer "B.Cu") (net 7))
 (segment (start 150.646513 99.695) (end 151.459338 98.882175) (width 0.25) (layer "B.Cu") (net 7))
 (segment (start 132.046055 98.829999) (end 133.87 98.829999) (width 0.25) (layer "F.Cu") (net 8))
 (segment (start 167.350291 86.705291) (end 167.350291 88.822774) (width 0.25) (layer "F.Cu") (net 8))
 (segment (start 166.318054 89.855011) (end 161.411616 89.855011) (width 0.25) (layer "F.Cu") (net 8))
 (segment (start 166.112403 90.060662) (end 166.318054 89.855011) (width 0.25) (layer "F.Cu") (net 8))
 (segment (start 133.87 98.829999) (end 134.62 98.079999) (width 0.25) (layer "F.Cu") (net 8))
 (segment (start 187.96 81.915) (end 187.96 84.98) (width 0.25) (layer "F.Cu") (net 8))
 (segment (start 167.350291 88.822774) (end 166.318054 89.855011) (width 0.25) (layer "F.Cu") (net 8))
 (segment (start 140.97 74.93) (end 128.455 87.445) (width 0.25) (layer "F.Cu") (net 8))
 (segment (start 166.583453 98.913275) (end 166.112403 98.442225) (width 0.25) (layer "F.Cu") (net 8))
 (segment (start 128.455 95.238944) (end 132.046055 98.829999) (width 0.25) (layer "F.Cu") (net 8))
 (segment (start 128.455 87.445) (end 128.455 95.238944) (width 0.25) (layer "F.Cu") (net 8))
 (segment (start 180.975 74.93) (end 187.96 81.915) (width 0.25) (layer "F.Cu") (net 8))
 (segment (start 155.575 74.93) (end 140.97 74.93) (width 0.25) (layer "F.Cu") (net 8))
 (segment (start 164.465 83.82) (end 167.350291 86.705291) (width 0.25) (layer "F.Cu") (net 8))
 (segment (start 166.112403 98.442225) (end 166.112403 90.060662) (width 0.25) (layer "F.Cu") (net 8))
 (segment (start 155.575 74.93) (end 164.465 83.82) (width 0.25) (layer "F.Cu") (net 8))
 (via (at 180.975 74.93) (size 0.8) (drill 0.4) (layers "F.Cu" "B.Cu") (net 8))
 (via (at 155.575 74.93) (size 0.8) (drill 0.4) (layers "F.Cu" "B.Cu") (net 8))
 (segment (start 155.575 74.93) (end 180.975 74.93) (width 0.25) (layer "B.Cu") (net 8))
 (segment (start 184.14975 76.20025) (end 191.96 84.0105) (width 0.25) (layer "F.Cu") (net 9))
 (segment (start 128.905 88.265) (end 128.905 95.052548) (width 0.25) (layer "F.Cu") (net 9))
 (segment (start 140.97 76.2) (end 128.905 88.265) (width 0.25) (layer "F.Cu") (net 9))
 (segment (start 162.743606 84.617608) (end 162.743606 85.866611) (width 0.25) (layer "F.Cu") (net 9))
 (segment (start 154.305 76.2) (end 154.325998 76.2) (width 0.25) (layer "F.Cu") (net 9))
 (segment (start 191.96 84.0105) (end 191.96 85.98) (width 0.25) (layer "F.Cu") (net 9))
 (segment (start 154.305 76.2) (end 140.97 76.2) (width 0.25) (layer "F.Cu") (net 9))
 (segment (start 154.325998 76.2) (end 162.743606 84.617608) (width 0.25) (layer "F.Cu") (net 9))
 (segment (start 128.905 95.052548) (end 131.149421 97.296969) (width 0.25) (layer "F.Cu") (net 9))
 (segment (start 131.149421 97.296969) (end 132.210081 97.296969) (width 0.25) (layer "F.Cu") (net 9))
 (via (at 184.14975 76.20025) (size 0.8) (drill 0.4) (layers "F.Cu" "B.Cu") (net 9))
 (via (at 154.305 76.2) (size 0.8) (drill 0.4) (layers "F.Cu" "B.Cu") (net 9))
 (segment (start 162.743606 85.866611) (end 159.39156 89.218657) (width 0.25) (layer "B.Cu") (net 9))
 (segment (start 184.14975 76.20025) (end 184.1495 76.2) (width 0.25) (layer "B.Cu") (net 9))
 (segment (start 184.1495 76.2) (end 154.305 76.2) (width 0.25) (layer "B.Cu") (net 9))
 (segment (start 159.39156 89.218657) (end 159.036716 89.218657) (width 0.25) (layer "B.Cu") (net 9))
 (segment (start 193.71 83.855) (end 193.71 89.48) (width 0.25) (layer "F.Cu") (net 10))
 (segment (start 156.845 81.28) (end 153.035 77.47) (width 0.25) (layer "F.Cu") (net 10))
 (segment (start 187.325 77.47) (end 193.71 83.855) (width 0.25) (layer "F.Cu") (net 10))
 (segment (start 129.645669 88.792935) (end 129.645669 94.171969) (width 0.25) (layer "F.Cu") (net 10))
 (segment (start 129.645669 94.171969) (end 130.720669 95.246969) (width 0.25) (layer "F.Cu") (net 10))
 (segment (start 153.035 77.47) (end 140.968604 77.47) (width 0.25) (layer "F.Cu") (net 10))
 (segment (start 140.968604 77.47) (end 129.645669 88.792935) (width 0.25) (layer "F.Cu") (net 10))
 (segment (start 156.845 83.185) (end 156.845 81.28) (width 0.25) (layer "F.Cu") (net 10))
 (via (at 187.325 77.47) (size 0.8) (drill 0.4) (layers "F.Cu" "B.Cu") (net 10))
 (via (at 153.035 77.47) (size 0.8) (drill 0.4) (layers "F.Cu" "B.Cu") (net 10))
 (via (at 156.845 83.185) (size 0.8) (drill 0.4) (layers "F.Cu" "B.Cu") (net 10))
 (segment (start 156.845 83.185) (end 164.465 83.185) (width 0.25) (layer "B.Cu") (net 10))
 (segment (start 156.845 83.185) (end 156.845 89.671827) (width 0.25) (layer "B.Cu") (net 10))
 (segment (start 156.845 89.671827) (end 156.661816 89.855011) (width 0.25) (layer "B.Cu") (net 10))
 (segment (start 164.465 83.185) (end 169.162403 87.882403) (width 0.25) (layer "B.Cu") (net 10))
 (segment (start 153.035 77.47) (end 187.325 77.47) (width 0.25) (layer "B.Cu") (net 10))
 (segment (start 169.162403 87.882403) (end 169.162403 94.042229) (width 0.25) (layer "B.Cu") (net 10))
 (segment (start 169.162403 94.042229) (end 167.914616 95.290016) (width 0.25) (layer "B.Cu") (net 10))
 (segment (start 131.266338 88.9) (end 130.720669 89.445669) (width 0.25) (layer "F.Cu") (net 11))
 (segment (start 151.765 78.74) (end 141.605 78.74) (width 0.25) (layer "F.Cu") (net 11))
 (segment (start 141.605 78.74) (end 131.445 88.9) (width 0.25) (layer "F.Cu") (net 11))
 (segment (start 131.445 88.9) (end 131.266338 88.9) (width 0.25) (layer "F.Cu") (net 11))
 (segment (start 195.58 83.91) (end 195.58 92.11) (width 0.25) (layer "F.Cu") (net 11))
 (segment (start 130.720669 89.445669) (end 130.720669 92.713031) (width 0.25) (layer "F.Cu") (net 11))
 (segment (start 190.52225 78.85225) (end 195.58 83.91) (width 0.25) (layer "F.Cu") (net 11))
 (segment (start 190.52225 78.71775) (end 190.52225 78.85225) (width 0.25) (layer "F.Cu") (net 11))
 (segment (start 151.765 78.74) (end 151.765 79.8123) (width 0.25) (layer "F.Cu") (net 11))
 (segment (start 195.58 92.11) (end 193.71 93.98) (width 0.25) (layer "F.Cu") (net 11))
 (segment (start 156.970246 87.391611) (end 165.025804 87.391611) (width 0.25) (layer "F.Cu") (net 11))
 (segment (start 156.768635 87.19) (end 156.970246 87.391611) (width 0.25) (layer "F.Cu") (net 11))
 (segment (start 151.765 79.8123) (end 156.768635 84.815935) (width 0.25) (layer "F.Cu") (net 11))
 (segment (start 156.768635 84.815935) (end 156.768635 87.19) (width 0.25) (layer "F.Cu") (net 11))
 (segment (start 154.92327 89.035364) (end 154.92327 91.593557) (width 0.25) (layer "F.Cu") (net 11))
 (segment (start 156.768635 87.19) (end 154.92327 89.035364) (width 0.25) (layer "F.Cu") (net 11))
 (segment (start 165.025804 87.391611) (end 165.825291 88.191098) (width 0.25) (layer "F.Cu") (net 11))
 (via (at 151.765 78.74) (size 0.8) (drill 0.4) (layers "F.Cu" "B.Cu") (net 11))
 (via (at 190.52225 78.71775) (size 0.8) (drill 0.4) (layers "F.Cu" "B.Cu") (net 11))
 (segment (start 151.765 78.74) (end 190.5 78.74) (width 0.25) (layer "B.Cu") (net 11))
 (segment (start 190.5 78.74) (end 190.52225 78.71775) (width 0.25) (layer "B.Cu") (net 11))
 (segment (start 150.495 80.01) (end 150.495 81.136276) (width 0.25) (layer "F.Cu") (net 2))
 (segment (start 196.85 83.185) (end 196.85 95.34) (width 0.25) (layer "F.Cu") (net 2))
 (segment (start 155.243635 87.326365) (end 153.50607 89.06393) (width 0.25) (layer "F.Cu") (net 2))
 (segment (start 196.85 95.34) (end 193.71 98.48) (width 0.25) (layer "F.Cu") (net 2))
 (segment (start 150.405 79.92) (end 142.953112 79.92) (width 0.25) (layer "F.Cu") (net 2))
 (segment (start 153.50607 89.06393) (end 153.50607 93.187611) (width 0.25) (layer "F.Cu") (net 2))
 (segment (start 155.243635 85.884911) (end 155.243635 87.326365) (width 0.25) (layer "F.Cu") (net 2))
 (segment (start 142.953112 79.92) (end 132.210081 90.663031) (width 0.25) (layer "F.Cu") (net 2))
 (segment (start 150.495 81.136276) (end 155.243635 85.884911) (width 0.25) (layer "F.Cu") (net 2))
 (segment (start 193.675 80.01) (end 196.85 83.185) (width 0.25) (layer "F.Cu") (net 2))
 (segment (start 153.50607 93.187611) (end 154.286916 93.968457) (width 0.25) (layer "F.Cu") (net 2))
 (segment (start 150.495 80.01) (end 150.405 79.92) (width 0.25) (layer "F.Cu") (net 2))
 (via (at 150.495 80.01) (size 0.8) (drill 0.4) (layers "F.Cu" "B.Cu") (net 2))
 (via (at 193.675 80.01) (size 0.8) (drill 0.4) (layers "F.Cu" "B.Cu") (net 2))
 (segment (start 193.675 80.01) (end 150.495 80.01) (width 0.25) (layer "B.Cu") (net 2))
 (segment (start 187.96 102.98) (end 187.96 114.28) (width 0.25) (layer "B.Cu") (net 13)))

